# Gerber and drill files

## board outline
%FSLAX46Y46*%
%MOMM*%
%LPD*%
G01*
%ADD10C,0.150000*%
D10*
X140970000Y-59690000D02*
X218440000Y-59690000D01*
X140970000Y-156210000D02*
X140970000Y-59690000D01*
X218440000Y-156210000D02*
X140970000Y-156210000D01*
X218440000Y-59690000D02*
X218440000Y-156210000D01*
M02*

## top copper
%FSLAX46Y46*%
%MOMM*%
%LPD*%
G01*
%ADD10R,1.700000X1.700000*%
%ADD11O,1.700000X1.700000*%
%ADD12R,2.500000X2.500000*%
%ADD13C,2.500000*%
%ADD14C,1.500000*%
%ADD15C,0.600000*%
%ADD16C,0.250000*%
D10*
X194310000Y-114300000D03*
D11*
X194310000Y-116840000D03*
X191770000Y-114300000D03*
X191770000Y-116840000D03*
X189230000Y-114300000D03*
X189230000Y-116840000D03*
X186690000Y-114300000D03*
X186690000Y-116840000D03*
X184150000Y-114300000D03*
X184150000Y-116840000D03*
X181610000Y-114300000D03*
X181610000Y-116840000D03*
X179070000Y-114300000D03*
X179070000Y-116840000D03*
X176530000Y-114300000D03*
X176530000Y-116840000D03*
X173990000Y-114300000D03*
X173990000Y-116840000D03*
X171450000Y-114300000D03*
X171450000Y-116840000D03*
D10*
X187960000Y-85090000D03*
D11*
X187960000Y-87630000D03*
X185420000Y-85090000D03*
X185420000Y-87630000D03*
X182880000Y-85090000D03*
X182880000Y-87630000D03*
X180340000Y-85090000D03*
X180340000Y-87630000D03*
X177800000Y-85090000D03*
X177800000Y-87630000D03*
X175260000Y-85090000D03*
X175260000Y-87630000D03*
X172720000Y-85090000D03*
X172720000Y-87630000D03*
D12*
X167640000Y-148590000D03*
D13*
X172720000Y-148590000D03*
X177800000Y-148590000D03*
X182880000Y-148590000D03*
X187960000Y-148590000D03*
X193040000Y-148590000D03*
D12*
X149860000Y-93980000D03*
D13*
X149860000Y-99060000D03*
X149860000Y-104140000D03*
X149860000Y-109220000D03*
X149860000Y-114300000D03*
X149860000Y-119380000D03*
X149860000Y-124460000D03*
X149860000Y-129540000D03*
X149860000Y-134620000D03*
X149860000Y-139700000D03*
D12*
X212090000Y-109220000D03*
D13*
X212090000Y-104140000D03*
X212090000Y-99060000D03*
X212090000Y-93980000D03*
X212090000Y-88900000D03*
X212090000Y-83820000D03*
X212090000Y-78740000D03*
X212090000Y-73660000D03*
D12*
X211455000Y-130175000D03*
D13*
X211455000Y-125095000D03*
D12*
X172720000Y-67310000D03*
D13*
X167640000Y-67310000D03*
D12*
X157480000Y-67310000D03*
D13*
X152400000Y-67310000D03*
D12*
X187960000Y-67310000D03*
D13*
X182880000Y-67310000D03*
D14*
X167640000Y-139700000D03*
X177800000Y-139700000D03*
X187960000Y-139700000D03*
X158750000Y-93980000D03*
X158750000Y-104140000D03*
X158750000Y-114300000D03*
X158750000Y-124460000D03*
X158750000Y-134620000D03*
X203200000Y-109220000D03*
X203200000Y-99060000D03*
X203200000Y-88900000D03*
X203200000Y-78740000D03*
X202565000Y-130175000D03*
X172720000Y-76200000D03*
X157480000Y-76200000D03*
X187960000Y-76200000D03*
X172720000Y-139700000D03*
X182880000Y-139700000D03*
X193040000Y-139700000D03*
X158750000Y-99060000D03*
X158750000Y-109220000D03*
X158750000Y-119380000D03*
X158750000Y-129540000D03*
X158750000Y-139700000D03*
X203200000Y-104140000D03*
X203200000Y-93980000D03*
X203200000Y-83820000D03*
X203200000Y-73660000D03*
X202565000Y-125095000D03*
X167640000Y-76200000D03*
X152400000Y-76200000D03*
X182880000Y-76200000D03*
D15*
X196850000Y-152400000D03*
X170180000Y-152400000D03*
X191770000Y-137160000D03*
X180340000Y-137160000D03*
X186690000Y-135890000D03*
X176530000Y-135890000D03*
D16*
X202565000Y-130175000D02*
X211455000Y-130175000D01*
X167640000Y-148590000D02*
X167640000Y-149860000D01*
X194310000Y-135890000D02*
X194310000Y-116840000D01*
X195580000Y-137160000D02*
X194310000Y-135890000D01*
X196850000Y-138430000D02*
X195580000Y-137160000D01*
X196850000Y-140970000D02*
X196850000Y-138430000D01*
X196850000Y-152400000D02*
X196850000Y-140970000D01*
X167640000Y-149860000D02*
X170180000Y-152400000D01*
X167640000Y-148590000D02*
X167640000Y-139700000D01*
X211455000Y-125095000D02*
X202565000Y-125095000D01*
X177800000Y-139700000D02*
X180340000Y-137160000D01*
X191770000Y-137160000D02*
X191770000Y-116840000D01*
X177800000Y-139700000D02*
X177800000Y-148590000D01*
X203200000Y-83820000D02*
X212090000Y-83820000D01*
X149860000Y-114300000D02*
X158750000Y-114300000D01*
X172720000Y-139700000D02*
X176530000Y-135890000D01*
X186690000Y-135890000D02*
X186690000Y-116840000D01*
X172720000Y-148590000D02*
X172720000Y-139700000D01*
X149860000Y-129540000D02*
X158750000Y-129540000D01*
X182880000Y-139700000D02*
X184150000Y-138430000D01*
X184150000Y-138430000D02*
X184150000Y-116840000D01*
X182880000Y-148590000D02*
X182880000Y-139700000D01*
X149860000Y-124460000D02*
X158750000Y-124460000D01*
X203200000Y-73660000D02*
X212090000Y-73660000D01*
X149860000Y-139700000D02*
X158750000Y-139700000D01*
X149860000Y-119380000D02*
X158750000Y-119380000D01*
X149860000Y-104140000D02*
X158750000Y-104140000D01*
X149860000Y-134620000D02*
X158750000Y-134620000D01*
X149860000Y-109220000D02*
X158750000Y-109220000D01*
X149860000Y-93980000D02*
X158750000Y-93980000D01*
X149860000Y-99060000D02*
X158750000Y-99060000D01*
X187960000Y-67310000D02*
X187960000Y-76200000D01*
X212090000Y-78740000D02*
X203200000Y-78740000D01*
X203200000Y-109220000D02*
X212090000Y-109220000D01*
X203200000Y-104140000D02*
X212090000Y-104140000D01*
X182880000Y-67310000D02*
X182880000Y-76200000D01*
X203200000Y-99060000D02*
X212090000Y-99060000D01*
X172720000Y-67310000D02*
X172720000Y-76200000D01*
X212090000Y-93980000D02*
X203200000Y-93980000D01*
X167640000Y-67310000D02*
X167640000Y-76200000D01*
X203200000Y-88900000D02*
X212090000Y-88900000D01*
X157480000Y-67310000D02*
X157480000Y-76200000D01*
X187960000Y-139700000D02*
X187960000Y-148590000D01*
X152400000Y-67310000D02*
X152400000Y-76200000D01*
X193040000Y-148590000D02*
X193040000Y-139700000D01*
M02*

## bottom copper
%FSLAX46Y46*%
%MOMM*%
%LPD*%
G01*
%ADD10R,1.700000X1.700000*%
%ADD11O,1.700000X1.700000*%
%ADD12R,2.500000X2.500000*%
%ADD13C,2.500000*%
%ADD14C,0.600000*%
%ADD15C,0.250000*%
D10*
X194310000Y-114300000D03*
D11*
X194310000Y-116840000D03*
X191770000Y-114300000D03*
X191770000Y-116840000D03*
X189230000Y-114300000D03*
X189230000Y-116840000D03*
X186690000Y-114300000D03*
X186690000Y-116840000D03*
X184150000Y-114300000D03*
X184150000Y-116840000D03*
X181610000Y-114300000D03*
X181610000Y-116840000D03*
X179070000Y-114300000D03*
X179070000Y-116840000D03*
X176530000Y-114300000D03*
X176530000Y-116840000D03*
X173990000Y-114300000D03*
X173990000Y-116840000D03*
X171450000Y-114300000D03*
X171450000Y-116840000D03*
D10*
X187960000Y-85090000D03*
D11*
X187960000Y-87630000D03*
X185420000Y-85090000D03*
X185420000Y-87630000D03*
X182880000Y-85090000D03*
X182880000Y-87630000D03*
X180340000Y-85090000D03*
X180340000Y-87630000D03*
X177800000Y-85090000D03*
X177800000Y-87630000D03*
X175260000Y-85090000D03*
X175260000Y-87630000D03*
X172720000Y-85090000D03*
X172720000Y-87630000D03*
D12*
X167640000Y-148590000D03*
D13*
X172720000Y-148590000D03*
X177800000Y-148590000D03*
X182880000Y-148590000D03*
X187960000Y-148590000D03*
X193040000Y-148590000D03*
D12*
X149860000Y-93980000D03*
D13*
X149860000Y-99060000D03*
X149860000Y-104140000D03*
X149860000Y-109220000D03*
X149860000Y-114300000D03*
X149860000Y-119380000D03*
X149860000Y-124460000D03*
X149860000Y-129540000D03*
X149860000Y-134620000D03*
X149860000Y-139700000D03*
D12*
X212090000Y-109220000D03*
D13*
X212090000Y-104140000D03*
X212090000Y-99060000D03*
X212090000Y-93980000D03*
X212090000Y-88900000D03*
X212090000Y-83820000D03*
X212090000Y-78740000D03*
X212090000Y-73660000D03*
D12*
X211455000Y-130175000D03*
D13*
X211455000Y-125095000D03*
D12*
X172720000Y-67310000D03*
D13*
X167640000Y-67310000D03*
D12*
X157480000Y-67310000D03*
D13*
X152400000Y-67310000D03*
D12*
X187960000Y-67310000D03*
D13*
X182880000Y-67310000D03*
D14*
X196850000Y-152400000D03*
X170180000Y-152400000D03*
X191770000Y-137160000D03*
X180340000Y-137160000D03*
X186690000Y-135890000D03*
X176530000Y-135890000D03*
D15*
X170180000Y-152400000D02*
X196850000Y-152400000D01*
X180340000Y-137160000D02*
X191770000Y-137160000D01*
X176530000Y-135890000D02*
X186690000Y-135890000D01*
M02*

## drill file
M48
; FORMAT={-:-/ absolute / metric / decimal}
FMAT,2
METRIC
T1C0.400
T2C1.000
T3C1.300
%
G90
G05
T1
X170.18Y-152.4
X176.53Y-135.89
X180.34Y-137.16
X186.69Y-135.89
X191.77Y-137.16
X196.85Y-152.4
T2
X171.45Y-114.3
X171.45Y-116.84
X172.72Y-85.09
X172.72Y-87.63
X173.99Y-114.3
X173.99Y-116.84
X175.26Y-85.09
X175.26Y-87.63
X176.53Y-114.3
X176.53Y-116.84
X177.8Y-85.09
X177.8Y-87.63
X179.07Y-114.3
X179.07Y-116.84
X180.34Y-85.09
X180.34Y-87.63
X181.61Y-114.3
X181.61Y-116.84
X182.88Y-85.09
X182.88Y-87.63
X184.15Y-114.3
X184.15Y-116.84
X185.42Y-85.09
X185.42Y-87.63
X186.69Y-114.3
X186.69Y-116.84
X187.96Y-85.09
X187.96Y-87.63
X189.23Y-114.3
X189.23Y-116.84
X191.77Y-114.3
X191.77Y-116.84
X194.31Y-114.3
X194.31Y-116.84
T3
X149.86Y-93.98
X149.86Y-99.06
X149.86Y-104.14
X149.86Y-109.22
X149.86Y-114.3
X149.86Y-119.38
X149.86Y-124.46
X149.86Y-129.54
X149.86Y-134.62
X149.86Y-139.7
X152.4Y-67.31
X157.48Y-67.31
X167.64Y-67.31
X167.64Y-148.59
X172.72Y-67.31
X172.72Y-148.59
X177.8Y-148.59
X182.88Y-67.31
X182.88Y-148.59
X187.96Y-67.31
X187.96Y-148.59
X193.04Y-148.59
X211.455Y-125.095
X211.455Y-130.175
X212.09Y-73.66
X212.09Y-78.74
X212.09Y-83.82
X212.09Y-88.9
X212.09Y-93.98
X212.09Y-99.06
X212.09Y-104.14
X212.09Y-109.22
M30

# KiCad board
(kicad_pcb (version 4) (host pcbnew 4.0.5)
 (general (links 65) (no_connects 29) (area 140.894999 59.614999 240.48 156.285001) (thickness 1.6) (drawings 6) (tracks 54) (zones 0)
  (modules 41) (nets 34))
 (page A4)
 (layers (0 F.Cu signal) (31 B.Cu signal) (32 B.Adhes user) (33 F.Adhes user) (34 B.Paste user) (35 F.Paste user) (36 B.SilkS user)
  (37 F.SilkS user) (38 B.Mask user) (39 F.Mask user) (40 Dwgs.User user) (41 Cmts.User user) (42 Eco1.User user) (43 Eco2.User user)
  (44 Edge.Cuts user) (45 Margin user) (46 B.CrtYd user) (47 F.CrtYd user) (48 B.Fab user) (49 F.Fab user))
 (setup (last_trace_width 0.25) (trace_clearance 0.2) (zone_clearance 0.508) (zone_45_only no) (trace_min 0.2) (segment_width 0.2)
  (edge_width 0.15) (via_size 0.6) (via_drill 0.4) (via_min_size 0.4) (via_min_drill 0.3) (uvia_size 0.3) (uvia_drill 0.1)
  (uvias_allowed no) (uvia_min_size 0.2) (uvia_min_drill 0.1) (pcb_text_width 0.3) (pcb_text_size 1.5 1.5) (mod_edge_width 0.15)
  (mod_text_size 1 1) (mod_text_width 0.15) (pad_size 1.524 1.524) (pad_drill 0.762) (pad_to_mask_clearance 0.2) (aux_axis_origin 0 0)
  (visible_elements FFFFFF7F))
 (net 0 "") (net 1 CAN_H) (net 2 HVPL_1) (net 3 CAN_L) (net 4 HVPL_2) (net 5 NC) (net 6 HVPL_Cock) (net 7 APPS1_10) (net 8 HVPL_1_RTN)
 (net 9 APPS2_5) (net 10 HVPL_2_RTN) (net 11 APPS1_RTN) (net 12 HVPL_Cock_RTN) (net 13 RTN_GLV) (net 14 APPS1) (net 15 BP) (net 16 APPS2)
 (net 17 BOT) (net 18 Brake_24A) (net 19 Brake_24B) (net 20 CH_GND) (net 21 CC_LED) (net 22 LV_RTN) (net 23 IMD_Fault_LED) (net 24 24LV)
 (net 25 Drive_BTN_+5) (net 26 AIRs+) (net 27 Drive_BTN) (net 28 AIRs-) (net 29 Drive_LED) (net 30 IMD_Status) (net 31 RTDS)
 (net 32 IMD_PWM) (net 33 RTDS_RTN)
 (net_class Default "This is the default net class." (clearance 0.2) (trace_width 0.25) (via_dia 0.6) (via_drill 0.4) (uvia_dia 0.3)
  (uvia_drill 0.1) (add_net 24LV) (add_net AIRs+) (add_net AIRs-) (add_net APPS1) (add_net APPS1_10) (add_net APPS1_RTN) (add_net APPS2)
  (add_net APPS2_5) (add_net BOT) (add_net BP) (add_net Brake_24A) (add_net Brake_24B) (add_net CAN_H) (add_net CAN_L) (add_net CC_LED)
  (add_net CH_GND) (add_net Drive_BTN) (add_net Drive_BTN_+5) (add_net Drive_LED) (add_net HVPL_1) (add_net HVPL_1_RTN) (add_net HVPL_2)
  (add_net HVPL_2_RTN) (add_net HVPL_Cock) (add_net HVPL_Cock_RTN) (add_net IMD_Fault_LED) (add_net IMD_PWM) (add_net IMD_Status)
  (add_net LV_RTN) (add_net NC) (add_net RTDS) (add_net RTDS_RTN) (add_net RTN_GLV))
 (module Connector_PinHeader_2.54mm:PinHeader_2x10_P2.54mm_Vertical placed (layer F.Cu) (at 194.31 114.3 270)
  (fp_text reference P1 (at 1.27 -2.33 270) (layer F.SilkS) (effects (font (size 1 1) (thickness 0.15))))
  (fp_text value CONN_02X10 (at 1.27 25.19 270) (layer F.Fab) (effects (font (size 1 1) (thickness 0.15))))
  (pad 1 thru_hole rect (at 0 0 270) (size 1.7 1.7) (drill 1) (layers *.Cu *.Mask) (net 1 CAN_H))
  (pad 2 thru_hole oval (at 2.54 0 270) (size 1.7 1.7) (drill 1) (layers *.Cu *.Mask) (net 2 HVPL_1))
  (pad 3 thru_hole oval (at 0 2.54 270) (size 1.7 1.7) (drill 1) (layers *.Cu *.Mask) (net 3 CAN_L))
  (pad 4 thru_hole oval (at 2.54 2.54 270) (size 1.7 1.7) (drill 1) (layers *.Cu *.Mask) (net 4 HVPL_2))
  (pad 5 thru_hole oval (at 0 5.08 270) (size 1.7 1.7) (drill 1) (layers *.Cu *.Mask) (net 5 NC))
  (pad 6 thru_hole oval (at 2.54 5.08 270) (size 1.7 1.7) (drill 1) (layers *.Cu *.Mask) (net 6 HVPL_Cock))
  (pad 7 thru_hole oval (at 0 7.62 270) (size 1.7 1.7) (drill 1) (layers *.Cu *.Mask) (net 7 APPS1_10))
  (pad 8 thru_hole oval (at 2.54 7.62 270) (size 1.7 1.7) (drill 1) (layers *.Cu *.Mask) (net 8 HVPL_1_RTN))
  (pad 9 thru_hole oval (at 0 10.16 270) (size 1.7 1.7) (drill 1) (layers *.Cu *.Mask) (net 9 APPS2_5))
  (pad 10 thru_hole oval (at 2.54 10.16 270) (size 1.7 1.7) (drill 1) (layers *.Cu *.Mask) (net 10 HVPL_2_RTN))
  (pad 11 thru_hole oval (at 0 12.7 270) (size 1.7 1.7) (drill 1) (layers *.Cu *.Mask) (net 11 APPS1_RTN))
  (pad 12 thru_hole oval (at 2.54 12.7 270) (size 1.7 1.7) (drill 1) (layers *.Cu *.Mask) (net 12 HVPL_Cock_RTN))
  (pad 13 thru_hole oval (at 0 15.24 270) (size 1.7 1.7) (drill 1) (layers *.Cu *.Mask) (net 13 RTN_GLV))
  (pad 14 thru_hole oval (at 2.54 15.24 270) (size 1.7 1.7) (drill 1) (layers *.Cu *.Mask) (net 5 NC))
  (pad 15 thru_hole oval (at 0 17.78 270) (size 1.7 1.7) (drill 1) (layers *.Cu *.Mask) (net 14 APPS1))
  (pad 16 thru_hole oval (at 2.54 17.78 270) (size 1.7 1.7) (drill 1) (layers *.Cu *.Mask) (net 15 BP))
  (pad 17 thru_hole oval (at 0 20.32 270) (size 1.7 1.7) (drill 1) (layers *.Cu *.Mask) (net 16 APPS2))
  (pad 18 thru_hole oval (at 2.54 20.32 270) (size 1.7 1.7) (drill 1) (layers *.Cu *.Mask) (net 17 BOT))
  (pad 19 thru_hole oval (at 0 22.86 270) (size 1.7 1.7) (drill 1) (layers *.Cu *.Mask) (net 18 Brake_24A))
  (pad 20 thru_hole oval (at 2.54 22.86 270) (size 1.7 1.7) (drill 1) (layers *.Cu *.Mask) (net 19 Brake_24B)))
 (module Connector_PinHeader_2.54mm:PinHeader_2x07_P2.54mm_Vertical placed (layer F.Cu) (at 187.96 85.09 270)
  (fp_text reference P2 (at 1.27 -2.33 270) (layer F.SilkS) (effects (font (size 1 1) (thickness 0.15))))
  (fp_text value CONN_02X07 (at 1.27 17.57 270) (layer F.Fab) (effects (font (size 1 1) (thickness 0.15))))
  (pad 1 thru_hole rect (at 0 0 270) (size 1.7 1.7) (drill 1) (layers *.Cu *.Mask) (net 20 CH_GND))
  (pad 2 thru_hole oval (at 2.54 0 270) (size 1.7 1.7) (drill 1) (layers *.Cu *.Mask) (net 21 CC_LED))
  (pad 3 thru_hole oval (at 0 2.54 270) (size 1.7 1.7) (drill 1) (layers *.Cu *.Mask) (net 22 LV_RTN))
  (pad 4 thru_hole oval (at 2.54 2.54 270) (size 1.7 1.7) (drill 1) (layers *.Cu *.Mask) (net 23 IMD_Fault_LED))
  (pad 5 thru_hole oval (at 0 5.08 270) (size 1.7 1.7) (drill 1) (layers *.Cu *.Mask) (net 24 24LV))
  (pad 6 thru_hole oval (at 2.54 5.08 270) (size 1.7 1.7) (drill 1) (layers *.Cu *.Mask) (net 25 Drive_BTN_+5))
  (pad 7 thru_hole oval (at 0 7.62 270) (size 1.7 1.7) (drill 1) (layers *.Cu *.Mask) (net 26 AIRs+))
  (pad 8 thru_hole oval (at 2.54 7.62 270) (size 1.7 1.7) (drill 1) (layers *.Cu *.Mask) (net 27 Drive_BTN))
  (pad 9 thru_hole oval (at 0 10.16 270) (size 1.7 1.7) (drill 1) (layers *.Cu *.Mask) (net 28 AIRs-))
  (pad 10 thru_hole oval (at 2.54 10.16 270) (size 1.7 1.7) (drill 1) (layers *.Cu *.Mask) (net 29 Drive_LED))
  (pad 11 thru_hole oval (at 0 12.7 270) (size 1.7 1.7) (drill 1) (layers *.Cu *.Mask) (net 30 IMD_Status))
  (pad 12 thru_hole oval (at 2.54 12.7 270) (size 1.7 1.7) (drill 1) (layers *.Cu *.Mask) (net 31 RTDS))
  (pad 13 thru_hole oval (at 0 15.24 270) (size 1.7 1.7) (drill 1) (layers *.Cu *.Mask) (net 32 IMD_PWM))
  (pad 14 thru_hole oval (at 2.54 15.24 270) (size 1.7 1.7) (drill 1) (layers *.Cu *.Mask) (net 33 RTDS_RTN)))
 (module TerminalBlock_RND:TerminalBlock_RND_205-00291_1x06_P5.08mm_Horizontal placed (layer F.Cu) (at 167.64 148.59)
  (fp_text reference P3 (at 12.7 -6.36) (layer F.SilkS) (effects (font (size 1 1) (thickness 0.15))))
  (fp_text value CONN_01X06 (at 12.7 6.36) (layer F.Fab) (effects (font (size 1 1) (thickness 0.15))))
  (pad 1 thru_hole rect (at 0 0) (size 2.5 2.5) (drill 1.3) (layers *.Cu *.Mask) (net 2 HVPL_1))
  (pad 2 thru_hole circle (at 5.08 0) (size 2.5 2.5) (drill 1.3) (layers *.Cu *.Mask) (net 8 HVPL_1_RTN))
  (pad 3 thru_hole circle (at 10.16 0) (size 2.5 2.5) (drill 1.3) (layers *.Cu *.Mask) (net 4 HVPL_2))
  (pad 4 thru_hole circle (at 15.24 0) (size 2.5 2.5) (drill 1.3) (layers *.Cu *.Mask) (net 10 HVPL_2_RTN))
  (pad 5 thru_hole circle (at 20.32 0) (size 2.5 2.5) (drill 1.3) (layers *.Cu *.Mask) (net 31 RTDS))
  (pad 6 thru_hole circle (at 25.4 0) (size 2.5 2.5) (drill 1.3) (layers *.Cu *.Mask) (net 33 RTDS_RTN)))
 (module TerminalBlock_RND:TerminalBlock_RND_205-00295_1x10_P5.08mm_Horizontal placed (layer F.Cu) (at 149.86 93.98 270)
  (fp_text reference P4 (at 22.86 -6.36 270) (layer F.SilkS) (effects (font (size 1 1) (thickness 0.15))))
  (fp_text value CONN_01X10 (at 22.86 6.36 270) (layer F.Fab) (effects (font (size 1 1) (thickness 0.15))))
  (pad 1 thru_hole rect (at 0 0 270) (size 2.5 2.5) (drill 1.3) (layers *.Cu *.Mask) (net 18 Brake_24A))
  (pad 2 thru_hole circle (at 5.08 0 270) (size 2.5 2.5) (drill 1.3) (layers *.Cu *.Mask) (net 19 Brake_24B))
  (pad 3 thru_hole circle (at 10.16 0 270) (size 2.5 2.5) (drill 1.3) (layers *.Cu *.Mask) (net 15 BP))
  (pad 4 thru_hole circle (at 15.24 0 270) (size 2.5 2.5) (drill 1.3) (layers *.Cu *.Mask) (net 17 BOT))
  (pad 5 thru_hole circle (at 20.32 0 270) (size 2.5 2.5) (drill 1.3) (layers *.Cu *.Mask) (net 7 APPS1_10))
  (pad 6 thru_hole circle (at 25.4 0 270) (size 2.5 2.5) (drill 1.3) (layers *.Cu *.Mask) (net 14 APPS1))
  (pad 7 thru_hole circle (at 30.48 0 270) (size 2.5 2.5) (drill 1.3) (layers *.Cu *.Mask) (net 11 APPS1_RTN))
  (pad 8 thru_hole circle (at 35.56 0 270) (size 2.5 2.5) (drill 1.3) (layers *.Cu *.Mask) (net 9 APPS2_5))
  (pad 9 thru_hole circle (at 40.64 0 270) (size 2.5 2.5) (drill 1.3) (layers *.Cu *.Mask) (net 16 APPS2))
  (pad 10 thru_hole circle (at 45.72 0 270) (size 2.5 2.5) (drill 1.3) (layers *.Cu *.Mask) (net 13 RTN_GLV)))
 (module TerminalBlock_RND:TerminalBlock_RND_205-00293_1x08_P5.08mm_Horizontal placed (layer F.Cu) (at 212.09 109.22 90)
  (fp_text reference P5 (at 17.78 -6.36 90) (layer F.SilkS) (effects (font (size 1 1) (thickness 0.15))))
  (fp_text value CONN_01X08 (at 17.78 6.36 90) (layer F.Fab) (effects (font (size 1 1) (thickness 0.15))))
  (pad 1 thru_hole rect (at 0 0 90) (size 2.5 2.5) (drill 1.3) (layers *.Cu *.Mask) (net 22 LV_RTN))
  (pad 2 thru_hole circle (at 5.08 0 90) (size 2.5 2.5) (drill 1.3) (layers *.Cu *.Mask) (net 23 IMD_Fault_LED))
  (pad 3 thru_hole circle (at 10.16 0 90) (size 2.5 2.5) (drill 1.3) (layers *.Cu *.Mask) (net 25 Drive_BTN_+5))
  (pad 4 thru_hole circle (at 15.24 0 90) (size 2.5 2.5) (drill 1.3) (layers *.Cu *.Mask) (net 27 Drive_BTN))
  (pad 5 thru_hole circle (at 20.32 0 90) (size 2.5 2.5) (drill 1.3) (layers *.Cu *.Mask) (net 29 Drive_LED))
  (pad 6 thru_hole circle (at 25.4 0 90) (size 2.5 2.5) (drill 1.3) (layers *.Cu *.Mask) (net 6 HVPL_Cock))
  (pad 7 thru_hole circle (at 30.48 0 90) (size 2.5 2.5) (drill 1.3) (layers *.Cu *.Mask) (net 21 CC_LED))
  (pad 8 thru_hole circle (at 35.56 0 90) (size 2.5 2.5) (drill 1.3) (layers *.Cu *.Mask) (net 12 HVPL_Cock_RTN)))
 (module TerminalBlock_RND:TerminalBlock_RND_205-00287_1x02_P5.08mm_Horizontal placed (layer F.Cu) (at 211.455 130.175 90)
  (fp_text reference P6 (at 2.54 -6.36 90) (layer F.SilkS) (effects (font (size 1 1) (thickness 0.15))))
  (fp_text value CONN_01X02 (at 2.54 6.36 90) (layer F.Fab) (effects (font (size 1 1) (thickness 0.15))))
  (pad 1 thru_hole rect (at 0 0 90) (size 2.5 2.5) (drill 1.3) (layers *.Cu *.Mask) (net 1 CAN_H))
  (pad 2 thru_hole circle (at 5.08 0 90) (size 2.5 2.5) (drill 1.3) (layers *.Cu *.Mask) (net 3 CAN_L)))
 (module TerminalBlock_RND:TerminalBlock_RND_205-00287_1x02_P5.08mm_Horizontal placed (layer F.Cu) (at 172.72 67.31 180)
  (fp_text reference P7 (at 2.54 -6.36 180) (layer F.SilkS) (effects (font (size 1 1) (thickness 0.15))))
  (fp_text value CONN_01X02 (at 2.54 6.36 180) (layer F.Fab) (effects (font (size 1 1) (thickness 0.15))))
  (pad 1 thru_hole rect (at 0 0 180) (size 2.5 2.5) (drill 1.3) (layers *.Cu *.Mask) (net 26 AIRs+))
  (pad 2 thru_hole circle (at 5.08 0 180) (size 2.5 2.5) (drill 1.3) (layers *.Cu *.Mask) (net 28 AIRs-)))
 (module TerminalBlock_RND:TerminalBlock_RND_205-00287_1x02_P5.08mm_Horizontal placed (layer F.Cu) (at 157.48 67.31 180)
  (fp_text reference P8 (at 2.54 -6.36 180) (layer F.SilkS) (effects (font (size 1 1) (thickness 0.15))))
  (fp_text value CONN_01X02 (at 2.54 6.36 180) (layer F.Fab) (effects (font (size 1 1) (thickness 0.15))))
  (pad 1 thru_hole rect (at 0 0 180) (size 2.5 2.5) (drill 1.3) (layers *.Cu *.Mask) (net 30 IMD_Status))
  (pad 2 thru_hole circle (at 5.08 0 180) (size 2.5 2.5) (drill 1.3) (layers *.Cu *.Mask) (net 32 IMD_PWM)))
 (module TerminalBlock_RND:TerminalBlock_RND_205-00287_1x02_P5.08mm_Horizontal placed (layer F.Cu) (at 187.96 67.31 180)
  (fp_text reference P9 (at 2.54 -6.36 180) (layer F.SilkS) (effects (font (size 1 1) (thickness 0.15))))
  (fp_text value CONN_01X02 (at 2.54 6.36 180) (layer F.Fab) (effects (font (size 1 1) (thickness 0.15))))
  (pad 1 thru_hole rect (at 0 0 180) (size 2.5 2.5) (drill 1.3) (layers *.Cu *.Mask) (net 20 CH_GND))
  (pad 2 thru_hole circle (at 5.08 0 180) (size 2.5 2.5) (drill 1.3) (layers *.Cu *.Mask) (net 24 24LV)))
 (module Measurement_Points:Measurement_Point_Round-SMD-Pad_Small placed (layer F.Cu) (at 167.64 139.7)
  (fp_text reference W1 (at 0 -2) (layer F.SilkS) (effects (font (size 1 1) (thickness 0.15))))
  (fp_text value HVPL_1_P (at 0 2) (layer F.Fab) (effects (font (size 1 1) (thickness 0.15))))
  (pad 1 smd circle (at 0 0) (size 1.5 1.5) (layers F.Cu F.Mask) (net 2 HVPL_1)))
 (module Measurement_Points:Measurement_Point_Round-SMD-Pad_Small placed (layer F.Cu) (at 177.8 139.7)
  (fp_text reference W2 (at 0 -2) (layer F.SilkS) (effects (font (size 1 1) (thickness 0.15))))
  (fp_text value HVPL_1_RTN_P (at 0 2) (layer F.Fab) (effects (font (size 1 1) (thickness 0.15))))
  (pad 1 smd circle (at 0 0) (size 1.5 1.5) (layers F.Cu F.Mask) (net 4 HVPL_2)))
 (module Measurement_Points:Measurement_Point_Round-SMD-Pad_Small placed (layer F.Cu) (at 187.96 139.7)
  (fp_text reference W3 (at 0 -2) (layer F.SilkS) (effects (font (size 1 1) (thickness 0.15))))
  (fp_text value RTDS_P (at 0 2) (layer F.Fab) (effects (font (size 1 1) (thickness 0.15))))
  (pad 1 smd circle (at 0 0) (size 1.5 1.5) (layers F.Cu F.Mask) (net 31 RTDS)))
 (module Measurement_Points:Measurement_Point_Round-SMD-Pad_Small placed (layer F.Cu) (at 158.75 93.98)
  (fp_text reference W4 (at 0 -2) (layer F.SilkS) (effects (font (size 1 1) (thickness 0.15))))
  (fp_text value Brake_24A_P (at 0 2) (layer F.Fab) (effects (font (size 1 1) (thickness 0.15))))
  (pad 1 smd circle (at 0 0) (size 1.5 1.5) (layers F.Cu F.Mask) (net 18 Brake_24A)))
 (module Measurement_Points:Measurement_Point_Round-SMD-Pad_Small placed (layer F.Cu) (at 158.75 104.14)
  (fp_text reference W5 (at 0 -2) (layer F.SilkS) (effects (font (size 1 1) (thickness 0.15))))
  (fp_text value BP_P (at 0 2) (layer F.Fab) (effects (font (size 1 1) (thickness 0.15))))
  (pad 1 smd circle (at 0 0) (size 1.5 1.5) (layers F.Cu F.Mask) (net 15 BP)))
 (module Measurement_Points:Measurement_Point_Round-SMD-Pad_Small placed (layer F.Cu) (at 158.75 114.3)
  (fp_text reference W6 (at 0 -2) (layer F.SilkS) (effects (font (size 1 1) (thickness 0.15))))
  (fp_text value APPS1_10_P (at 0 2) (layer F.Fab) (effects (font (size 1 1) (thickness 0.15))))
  (pad 1 smd circle (at 0 0) (size 1.5 1.5) (layers F.Cu F.Mask) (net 7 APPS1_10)))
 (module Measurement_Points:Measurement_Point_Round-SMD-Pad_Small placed (layer F.Cu) (at 158.75 124.46)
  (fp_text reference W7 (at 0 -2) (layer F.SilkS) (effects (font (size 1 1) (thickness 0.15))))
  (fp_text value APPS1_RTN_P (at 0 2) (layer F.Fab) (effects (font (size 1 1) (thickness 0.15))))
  (pad 1 smd circle (at 0 0) (size 1.5 1.5) (layers F.Cu F.Mask) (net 11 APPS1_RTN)))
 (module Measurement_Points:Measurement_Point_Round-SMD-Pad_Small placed (layer F.Cu) (at 158.75 134.62)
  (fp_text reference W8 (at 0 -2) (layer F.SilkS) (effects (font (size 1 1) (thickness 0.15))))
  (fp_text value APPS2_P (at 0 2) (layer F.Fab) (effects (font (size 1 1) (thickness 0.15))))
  (pad 1 smd circle (at 0 0) (size 1.5 1.5) (layers F.Cu F.Mask) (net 16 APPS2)))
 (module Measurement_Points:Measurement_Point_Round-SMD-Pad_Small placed (layer F.Cu) (at 203.2 109.22)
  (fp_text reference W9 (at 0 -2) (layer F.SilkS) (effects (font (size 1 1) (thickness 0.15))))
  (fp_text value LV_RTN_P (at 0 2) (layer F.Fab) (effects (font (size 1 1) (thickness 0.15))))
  (pad 1 smd circle (at 0 0) (size 1.5 1.5) (layers F.Cu F.Mask) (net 22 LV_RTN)))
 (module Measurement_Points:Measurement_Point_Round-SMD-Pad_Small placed (layer F.Cu) (at 203.2 99.06)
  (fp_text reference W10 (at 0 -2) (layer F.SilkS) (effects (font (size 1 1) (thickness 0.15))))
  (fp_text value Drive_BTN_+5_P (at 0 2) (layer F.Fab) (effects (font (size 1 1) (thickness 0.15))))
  (pad 1 smd circle (at 0 0) (size 1.5 1.5) (layers F.Cu F.Mask) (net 25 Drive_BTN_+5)))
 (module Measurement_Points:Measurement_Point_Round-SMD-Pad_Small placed (layer F.Cu) (at 203.2 88.9)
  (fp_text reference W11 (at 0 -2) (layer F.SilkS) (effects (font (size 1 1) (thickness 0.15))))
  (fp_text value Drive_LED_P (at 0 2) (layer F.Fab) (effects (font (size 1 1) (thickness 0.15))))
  (pad 1 smd circle (at 0 0) (size 1.5 1.5) (layers F.Cu F.Mask) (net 29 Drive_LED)))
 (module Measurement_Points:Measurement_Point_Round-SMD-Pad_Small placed (layer F.Cu) (at 203.2 78.74)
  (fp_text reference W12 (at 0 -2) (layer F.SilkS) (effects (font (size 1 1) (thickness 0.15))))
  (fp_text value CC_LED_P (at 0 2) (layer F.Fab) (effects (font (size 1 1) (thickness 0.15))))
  (pad 1 smd circle (at 0 0) (size 1.5 1.5) (layers F.Cu F.Mask) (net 21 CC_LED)))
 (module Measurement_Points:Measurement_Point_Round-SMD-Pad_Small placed (layer F.Cu) (at 202.565 130.175 180)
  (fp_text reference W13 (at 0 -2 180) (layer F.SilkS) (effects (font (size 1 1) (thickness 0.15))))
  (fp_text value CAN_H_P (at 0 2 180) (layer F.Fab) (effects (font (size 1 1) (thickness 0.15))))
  (pad 1 smd circle (at 0 0 180) (size 1.5 1.5) (layers F.Cu F.Mask) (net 1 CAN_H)))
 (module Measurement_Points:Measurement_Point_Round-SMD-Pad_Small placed (layer F.Cu) (at 172.72 76.2 90)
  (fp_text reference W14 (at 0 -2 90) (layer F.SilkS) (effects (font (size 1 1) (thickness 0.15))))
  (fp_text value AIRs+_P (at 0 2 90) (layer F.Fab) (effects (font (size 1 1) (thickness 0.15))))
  (pad 1 smd circle (at 0 0 90) (size 1.5 1.5) (layers F.Cu F.Mask) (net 26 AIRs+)))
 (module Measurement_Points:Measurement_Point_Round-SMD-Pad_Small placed (layer F.Cu) (at 157.48 76.2)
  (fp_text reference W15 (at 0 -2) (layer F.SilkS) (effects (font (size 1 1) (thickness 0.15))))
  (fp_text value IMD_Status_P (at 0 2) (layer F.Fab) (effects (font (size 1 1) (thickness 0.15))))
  (pad 1 smd circle (at 0 0) (size 1.5 1.5) (layers F.Cu F.Mask) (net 30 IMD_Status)))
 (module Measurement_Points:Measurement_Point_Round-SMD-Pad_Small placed (layer F.Cu) (at 187.96 76.2)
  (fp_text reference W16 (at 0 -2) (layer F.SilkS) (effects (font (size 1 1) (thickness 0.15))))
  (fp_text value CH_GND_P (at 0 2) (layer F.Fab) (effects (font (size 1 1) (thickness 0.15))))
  (pad 1 smd circle (at 0 0) (size 1.5 1.5) (layers F.Cu F.Mask) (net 20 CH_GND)))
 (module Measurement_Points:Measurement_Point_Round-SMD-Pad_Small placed (layer F.Cu) (at 172.72 139.7)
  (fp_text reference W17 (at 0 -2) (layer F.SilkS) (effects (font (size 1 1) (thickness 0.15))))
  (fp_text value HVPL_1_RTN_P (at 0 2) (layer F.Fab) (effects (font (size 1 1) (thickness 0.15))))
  (pad 1 smd circle (at 0 0) (size 1.5 1.5) (layers F.Cu F.Mask) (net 8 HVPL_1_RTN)))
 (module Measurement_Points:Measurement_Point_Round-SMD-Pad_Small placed (layer F.Cu) (at 182.88 139.7)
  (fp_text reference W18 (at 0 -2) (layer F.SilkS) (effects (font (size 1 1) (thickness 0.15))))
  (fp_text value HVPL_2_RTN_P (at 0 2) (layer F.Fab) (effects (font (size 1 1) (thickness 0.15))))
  (pad 1 smd circle (at 0 0) (size 1.5 1.5) (layers F.Cu F.Mask) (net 10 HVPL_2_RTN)))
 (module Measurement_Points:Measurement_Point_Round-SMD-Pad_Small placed (layer F.Cu) (at 193.04 139.7)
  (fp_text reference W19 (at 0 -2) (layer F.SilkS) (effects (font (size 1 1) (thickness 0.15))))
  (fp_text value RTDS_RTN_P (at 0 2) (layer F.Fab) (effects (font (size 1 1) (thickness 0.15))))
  (pad 1 smd circle (at 0 0) (size 1.5 1.5) (layers F.Cu F.Mask) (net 33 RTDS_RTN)))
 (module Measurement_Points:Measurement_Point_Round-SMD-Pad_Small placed (layer F.Cu) (at 158.75 99.06)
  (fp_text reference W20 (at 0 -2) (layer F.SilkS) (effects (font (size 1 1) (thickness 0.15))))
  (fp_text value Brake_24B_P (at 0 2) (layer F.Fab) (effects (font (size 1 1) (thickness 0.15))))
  (pad 1 smd circle (at 0 0) (size 1.5 1.5) (layers F.Cu F.Mask) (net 19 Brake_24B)))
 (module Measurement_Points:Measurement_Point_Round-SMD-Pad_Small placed (layer F.Cu) (at 158.75 109.22)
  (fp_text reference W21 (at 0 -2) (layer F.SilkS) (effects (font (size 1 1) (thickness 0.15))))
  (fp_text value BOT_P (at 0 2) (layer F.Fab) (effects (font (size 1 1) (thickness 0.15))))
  (pad 1 smd circle (at 0 0) (size 1.5 1.5) (layers F.Cu F.Mask) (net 17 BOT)))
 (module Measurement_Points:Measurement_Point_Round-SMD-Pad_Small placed (layer F.Cu) (at 158.75 119.38)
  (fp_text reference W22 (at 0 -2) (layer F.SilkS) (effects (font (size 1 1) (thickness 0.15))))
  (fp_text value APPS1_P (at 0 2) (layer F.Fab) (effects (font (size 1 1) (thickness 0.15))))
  (pad 1 smd circle (at 0 0) (size 1.5 1.5) (layers F.Cu F.Mask) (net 14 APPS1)))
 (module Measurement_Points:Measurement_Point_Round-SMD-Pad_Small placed (layer F.Cu) (at 158.75 129.54)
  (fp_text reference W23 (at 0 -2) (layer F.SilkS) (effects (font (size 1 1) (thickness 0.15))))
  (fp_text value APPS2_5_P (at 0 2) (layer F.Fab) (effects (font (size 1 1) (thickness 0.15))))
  (pad 1 smd circle (at 0 0) (size 1.5 1.5) (layers F.Cu F.Mask) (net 9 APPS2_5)))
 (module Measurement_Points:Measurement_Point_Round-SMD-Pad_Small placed (layer F.Cu) (at 158.75 139.7)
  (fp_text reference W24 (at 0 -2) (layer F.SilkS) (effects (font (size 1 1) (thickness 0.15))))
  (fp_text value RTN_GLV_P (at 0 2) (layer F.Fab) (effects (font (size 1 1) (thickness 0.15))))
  (pad 1 smd circle (at 0 0) (size 1.5 1.5) (layers F.Cu F.Mask) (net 13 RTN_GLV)))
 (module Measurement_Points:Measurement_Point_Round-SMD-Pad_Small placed (layer F.Cu) (at 203.2 104.14)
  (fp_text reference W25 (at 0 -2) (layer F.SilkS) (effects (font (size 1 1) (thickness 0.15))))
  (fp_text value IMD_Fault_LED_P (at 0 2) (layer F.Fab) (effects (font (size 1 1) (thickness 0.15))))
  (pad 1 smd circle (at 0 0) (size 1.5 1.5) (layers F.Cu F.Mask) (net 23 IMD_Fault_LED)))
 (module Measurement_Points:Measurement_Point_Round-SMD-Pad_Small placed (layer F.Cu) (at 203.2 93.98)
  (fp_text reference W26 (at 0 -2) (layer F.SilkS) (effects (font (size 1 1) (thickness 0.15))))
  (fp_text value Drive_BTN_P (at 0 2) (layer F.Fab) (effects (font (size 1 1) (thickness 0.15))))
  (pad 1 smd circle (at 0 0) (size 1.5 1.5) (layers F.Cu F.Mask) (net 27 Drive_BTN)))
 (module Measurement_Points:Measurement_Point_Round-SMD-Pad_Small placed (layer F.Cu) (at 203.2 83.82)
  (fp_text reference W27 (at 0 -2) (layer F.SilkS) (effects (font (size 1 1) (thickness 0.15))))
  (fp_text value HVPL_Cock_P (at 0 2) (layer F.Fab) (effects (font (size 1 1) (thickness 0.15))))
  (pad 1 smd circle (at 0 0) (size 1.5 1.5) (layers F.Cu F.Mask) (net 6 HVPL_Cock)))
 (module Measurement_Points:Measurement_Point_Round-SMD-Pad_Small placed (layer F.Cu) (at 203.2 73.66)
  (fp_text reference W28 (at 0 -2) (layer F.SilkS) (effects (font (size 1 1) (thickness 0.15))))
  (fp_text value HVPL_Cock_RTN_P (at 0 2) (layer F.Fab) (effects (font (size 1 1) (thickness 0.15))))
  (pad 1 smd circle (at 0 0) (size 1.5 1.5) (layers F.Cu F.Mask) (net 12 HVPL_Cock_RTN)))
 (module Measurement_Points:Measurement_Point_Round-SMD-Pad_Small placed (layer F.Cu) (at 202.565 125.095 180)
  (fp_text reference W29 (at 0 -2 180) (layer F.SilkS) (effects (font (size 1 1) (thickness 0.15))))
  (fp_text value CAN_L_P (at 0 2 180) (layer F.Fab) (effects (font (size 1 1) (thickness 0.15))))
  (pad 1 smd circle (at 0 0 180) (size 1.5 1.5) (layers F.Cu F.Mask) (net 3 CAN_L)))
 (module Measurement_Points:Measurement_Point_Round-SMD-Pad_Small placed (layer F.Cu) (at 167.64 76.2 90)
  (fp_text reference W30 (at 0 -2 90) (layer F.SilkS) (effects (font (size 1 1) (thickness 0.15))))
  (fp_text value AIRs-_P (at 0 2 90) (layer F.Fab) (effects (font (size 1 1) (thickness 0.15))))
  (pad 1 smd circle (at 0 0 90) (size 1.5 1.5) (layers F.Cu F.Mask) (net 28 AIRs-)))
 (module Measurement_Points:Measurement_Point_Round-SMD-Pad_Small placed (layer F.Cu) (at 152.4 76.2)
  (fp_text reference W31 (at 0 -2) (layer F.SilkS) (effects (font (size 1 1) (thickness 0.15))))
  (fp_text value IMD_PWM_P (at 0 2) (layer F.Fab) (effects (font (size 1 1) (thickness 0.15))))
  (pad 1 smd circle (at 0 0) (size 1.5 1.5) (layers F.Cu F.Mask) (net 32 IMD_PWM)))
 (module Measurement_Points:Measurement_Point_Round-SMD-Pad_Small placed (layer F.Cu) (at 182.88 76.2)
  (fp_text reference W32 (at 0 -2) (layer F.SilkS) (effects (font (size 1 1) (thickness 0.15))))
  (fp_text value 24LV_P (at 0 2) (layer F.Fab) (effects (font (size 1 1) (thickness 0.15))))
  (pad 1 smd circle (at 0 0) (size 1.5 1.5) (layers F.Cu F.Mask) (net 24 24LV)))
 (gr_line (start 140.97 59.69) (end 218.44 59.69) (angle 90) (layer Edge.Cuts) (width 0.15))
 (gr_line (start 140.97 156.21) (end 140.97 59.69) (angle 90) (layer Edge.Cuts) (width 0.15))
 (gr_line (start 218.44 156.21) (end 140.97 156.21) (angle 90) (layer Edge.Cuts) (width 0.15))
 (gr_line (start 218.44 59.69) (end 218.44 156.21) (angle 90) (layer Edge.Cuts) (width 0.15))
 (segment (start 202.565 130.175) (end 211.455 130.175) (width 0.25) (layer F.Cu) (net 1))
 (segment (start 167.64 148.59) (end 167.64 149.86) (width 0.25) (layer F.Cu) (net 2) (status 400000))
 (segment (start 194.31 135.89) (end 194.31 116.84) (width 0.25) (layer F.Cu) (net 2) (status 800000))
 (segment (start 195.58 137.16) (end 194.31 135.89) (width 0.25) (layer F.Cu) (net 2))
 (segment (start 196.85 138.43) (end 195.58 137.16) (width 0.25) (layer F.Cu) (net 2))
 (segment (start 196.85 140.97) (end 196.85 138.43) (width 0.25) (layer F.Cu) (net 2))
 (segment (start 196.85 152.4) (end 196.85 140.97) (width 0.25) (layer F.Cu) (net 2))
 (via (at 196.85 152.4) (size 0.6) (drill 0.4) (layers F.Cu B.Cu) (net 2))
 (segment (start 170.18 152.4) (end 196.85 152.4) (width 0.25) (layer B.Cu) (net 2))
 (via (at 170.18 152.4) (size 0.6) (drill 0.4) (layers F.Cu B.Cu) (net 2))
 (segment (start 167.64 149.86) (end 170.18 152.4) (width 0.25) (layer F.Cu) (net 2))
 (segment (start 167.64 148.59) (end 167.64 139.7) (width 0.25) (layer F.Cu) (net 2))
 (segment (start 211.455 125.095) (end 202.565 125.095) (width 0.25) (layer F.Cu) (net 3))
 (segment (start 177.8 139.7) (end 180.34 137.16) (width 0.25) (layer F.Cu) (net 4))
 (segment (start 191.77 137.16) (end 191.77 116.84) (width 0.25) (layer F.Cu) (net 4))
 (via (at 191.77 137.16) (size 0.6) (drill 0.4) (layers F.Cu B.Cu) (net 4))
 (segment (start 180.34 137.16) (end 191.77 137.16) (width 0.25) (layer B.Cu) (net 4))
 (via (at 180.34 137.16) (size 0.6) (drill 0.4) (layers F.Cu B.Cu) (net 4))
 (segment (start 177.8 139.7) (end 177.8 148.59) (width 0.25) (layer F.Cu) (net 4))
 (segment (start 203.2 83.82) (end 212.09 83.82) (width 0.25) (layer F.Cu) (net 6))
 (segment (start 149.86 114.3) (end 158.75 114.3) (width 0.25) (layer F.Cu) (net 7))
 (segment (start 172.72 139.7) (end 176.53 135.89) (width 0.25) (layer F.Cu) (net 8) (status 400000))
 (segment (start 186.69 135.89) (end 186.69 116.84) (width 0.25) (layer F.Cu) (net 8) (status 800000))
 (via (at 186.69 135.89) (size 0.6) (drill 0.4) (layers F.Cu B.Cu) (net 8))
 (segment (start 176.53 135.89) (end 186.69 135.89) (width 0.25) (layer B.Cu) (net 8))
 (via (at 176.53 135.89) (size 0.6) (drill 0.4) (layers F.Cu B.Cu) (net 8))
 (segment (start 172.72 148.59) (end 172.72 139.7) (width 0.25) (layer F.Cu) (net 8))
 (segment (start 149.86 129.54) (end 158.75 129.54) (width 0.25) (layer F.Cu) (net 9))
 (segment (start 182.88 139.7) (end 184.15 138.43) (width 0.25) (layer F.Cu) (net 10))
 (segment (start 184.15 138.43) (end 184.15 116.84) (width 0.25) (layer F.Cu) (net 10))
 (segment (start 182.88 148.59) (end 182.88 139.7) (width 0.25) (layer F.Cu) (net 10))
 (segment (start 149.86 124.46) (end 158.75 124.46) (width 0.25) (layer F.Cu) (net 11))
 (segment (start 203.2 73.66) (end 212.09 73.66) (width 0.25) (layer F.Cu) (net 12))
 (segment (start 149.86 139.7) (end 158.75 139.7) (width 0.25) (layer F.Cu) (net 13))
 (segment (start 149.86 119.38) (end 158.75 119.38) (width 0.25) (layer F.Cu) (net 14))
 (segment (start 149.86 104.14) (end 158.75 104.14) (width 0.25) (layer F.Cu) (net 15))
 (segment (start 149.86 134.62) (end 158.75 134.62) (width 0.25) (layer F.Cu) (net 16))
 (segment (start 149.86 109.22) (end 158.75 109.22) (width 0.25) (layer F.Cu) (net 17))
 (segment (start 149.86 93.98) (end 158.75 93.98) (width 0.25) (layer F.Cu) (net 18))
 (segment (start 149.86 99.06) (end 158.75 99.06) (width 0.25) (layer F.Cu) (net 19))
 (segment (start 187.96 67.31) (end 187.96 76.2) (width 0.25) (layer F.Cu) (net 20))
 (segment (start 212.09 78.74) (end 203.2 78.74) (width 0.25) (layer F.Cu) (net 21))
 (segment (start 203.2 109.22) (end 212.09 109.22) (width 0.25) (layer F.Cu) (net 22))
 (segment (start 203.2 104.14) (end 212.09 104.14) (width 0.25) (layer F.Cu) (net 23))
 (segment (start 182.88 67.31) (end 182.88 76.2) (width 0.25) (layer F.Cu) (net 24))
 (segment (start 203.2 99.06) (end 212.09 99.06) (width 0.25) (layer F.Cu) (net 25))
 (segment (start 172.72 67.31) (end 172.72 76.2) (width 0.25) (layer F.Cu) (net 26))
 (segment (start 212.09 93.98) (end 203.2 93.98) (width 0.25) (layer F.Cu) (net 27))
 (segment (start 167.64 67.31) (end 167.64 76.2) (width 0.25) (layer F.Cu) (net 28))
 (segment (start 203.2 88.9) (end 212.09 88.9) (width 0.25) (layer F.Cu) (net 29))
 (segment (start 157.48 67.31) (end 157.48 76.2) (width 0.25) (layer F.Cu) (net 30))
 (segment (start 187.96 139.7) (end 187.96 148.59) (width 0.25) (layer F.Cu) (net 31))
 (segment (start 152.4 67.31) (end 152.4 76.2) (width 0.25) (layer F.Cu) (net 32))
 (segment (start 193.04 148.59) (end 193.04 139.7) (width 0.25) (layer F.Cu) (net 33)))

